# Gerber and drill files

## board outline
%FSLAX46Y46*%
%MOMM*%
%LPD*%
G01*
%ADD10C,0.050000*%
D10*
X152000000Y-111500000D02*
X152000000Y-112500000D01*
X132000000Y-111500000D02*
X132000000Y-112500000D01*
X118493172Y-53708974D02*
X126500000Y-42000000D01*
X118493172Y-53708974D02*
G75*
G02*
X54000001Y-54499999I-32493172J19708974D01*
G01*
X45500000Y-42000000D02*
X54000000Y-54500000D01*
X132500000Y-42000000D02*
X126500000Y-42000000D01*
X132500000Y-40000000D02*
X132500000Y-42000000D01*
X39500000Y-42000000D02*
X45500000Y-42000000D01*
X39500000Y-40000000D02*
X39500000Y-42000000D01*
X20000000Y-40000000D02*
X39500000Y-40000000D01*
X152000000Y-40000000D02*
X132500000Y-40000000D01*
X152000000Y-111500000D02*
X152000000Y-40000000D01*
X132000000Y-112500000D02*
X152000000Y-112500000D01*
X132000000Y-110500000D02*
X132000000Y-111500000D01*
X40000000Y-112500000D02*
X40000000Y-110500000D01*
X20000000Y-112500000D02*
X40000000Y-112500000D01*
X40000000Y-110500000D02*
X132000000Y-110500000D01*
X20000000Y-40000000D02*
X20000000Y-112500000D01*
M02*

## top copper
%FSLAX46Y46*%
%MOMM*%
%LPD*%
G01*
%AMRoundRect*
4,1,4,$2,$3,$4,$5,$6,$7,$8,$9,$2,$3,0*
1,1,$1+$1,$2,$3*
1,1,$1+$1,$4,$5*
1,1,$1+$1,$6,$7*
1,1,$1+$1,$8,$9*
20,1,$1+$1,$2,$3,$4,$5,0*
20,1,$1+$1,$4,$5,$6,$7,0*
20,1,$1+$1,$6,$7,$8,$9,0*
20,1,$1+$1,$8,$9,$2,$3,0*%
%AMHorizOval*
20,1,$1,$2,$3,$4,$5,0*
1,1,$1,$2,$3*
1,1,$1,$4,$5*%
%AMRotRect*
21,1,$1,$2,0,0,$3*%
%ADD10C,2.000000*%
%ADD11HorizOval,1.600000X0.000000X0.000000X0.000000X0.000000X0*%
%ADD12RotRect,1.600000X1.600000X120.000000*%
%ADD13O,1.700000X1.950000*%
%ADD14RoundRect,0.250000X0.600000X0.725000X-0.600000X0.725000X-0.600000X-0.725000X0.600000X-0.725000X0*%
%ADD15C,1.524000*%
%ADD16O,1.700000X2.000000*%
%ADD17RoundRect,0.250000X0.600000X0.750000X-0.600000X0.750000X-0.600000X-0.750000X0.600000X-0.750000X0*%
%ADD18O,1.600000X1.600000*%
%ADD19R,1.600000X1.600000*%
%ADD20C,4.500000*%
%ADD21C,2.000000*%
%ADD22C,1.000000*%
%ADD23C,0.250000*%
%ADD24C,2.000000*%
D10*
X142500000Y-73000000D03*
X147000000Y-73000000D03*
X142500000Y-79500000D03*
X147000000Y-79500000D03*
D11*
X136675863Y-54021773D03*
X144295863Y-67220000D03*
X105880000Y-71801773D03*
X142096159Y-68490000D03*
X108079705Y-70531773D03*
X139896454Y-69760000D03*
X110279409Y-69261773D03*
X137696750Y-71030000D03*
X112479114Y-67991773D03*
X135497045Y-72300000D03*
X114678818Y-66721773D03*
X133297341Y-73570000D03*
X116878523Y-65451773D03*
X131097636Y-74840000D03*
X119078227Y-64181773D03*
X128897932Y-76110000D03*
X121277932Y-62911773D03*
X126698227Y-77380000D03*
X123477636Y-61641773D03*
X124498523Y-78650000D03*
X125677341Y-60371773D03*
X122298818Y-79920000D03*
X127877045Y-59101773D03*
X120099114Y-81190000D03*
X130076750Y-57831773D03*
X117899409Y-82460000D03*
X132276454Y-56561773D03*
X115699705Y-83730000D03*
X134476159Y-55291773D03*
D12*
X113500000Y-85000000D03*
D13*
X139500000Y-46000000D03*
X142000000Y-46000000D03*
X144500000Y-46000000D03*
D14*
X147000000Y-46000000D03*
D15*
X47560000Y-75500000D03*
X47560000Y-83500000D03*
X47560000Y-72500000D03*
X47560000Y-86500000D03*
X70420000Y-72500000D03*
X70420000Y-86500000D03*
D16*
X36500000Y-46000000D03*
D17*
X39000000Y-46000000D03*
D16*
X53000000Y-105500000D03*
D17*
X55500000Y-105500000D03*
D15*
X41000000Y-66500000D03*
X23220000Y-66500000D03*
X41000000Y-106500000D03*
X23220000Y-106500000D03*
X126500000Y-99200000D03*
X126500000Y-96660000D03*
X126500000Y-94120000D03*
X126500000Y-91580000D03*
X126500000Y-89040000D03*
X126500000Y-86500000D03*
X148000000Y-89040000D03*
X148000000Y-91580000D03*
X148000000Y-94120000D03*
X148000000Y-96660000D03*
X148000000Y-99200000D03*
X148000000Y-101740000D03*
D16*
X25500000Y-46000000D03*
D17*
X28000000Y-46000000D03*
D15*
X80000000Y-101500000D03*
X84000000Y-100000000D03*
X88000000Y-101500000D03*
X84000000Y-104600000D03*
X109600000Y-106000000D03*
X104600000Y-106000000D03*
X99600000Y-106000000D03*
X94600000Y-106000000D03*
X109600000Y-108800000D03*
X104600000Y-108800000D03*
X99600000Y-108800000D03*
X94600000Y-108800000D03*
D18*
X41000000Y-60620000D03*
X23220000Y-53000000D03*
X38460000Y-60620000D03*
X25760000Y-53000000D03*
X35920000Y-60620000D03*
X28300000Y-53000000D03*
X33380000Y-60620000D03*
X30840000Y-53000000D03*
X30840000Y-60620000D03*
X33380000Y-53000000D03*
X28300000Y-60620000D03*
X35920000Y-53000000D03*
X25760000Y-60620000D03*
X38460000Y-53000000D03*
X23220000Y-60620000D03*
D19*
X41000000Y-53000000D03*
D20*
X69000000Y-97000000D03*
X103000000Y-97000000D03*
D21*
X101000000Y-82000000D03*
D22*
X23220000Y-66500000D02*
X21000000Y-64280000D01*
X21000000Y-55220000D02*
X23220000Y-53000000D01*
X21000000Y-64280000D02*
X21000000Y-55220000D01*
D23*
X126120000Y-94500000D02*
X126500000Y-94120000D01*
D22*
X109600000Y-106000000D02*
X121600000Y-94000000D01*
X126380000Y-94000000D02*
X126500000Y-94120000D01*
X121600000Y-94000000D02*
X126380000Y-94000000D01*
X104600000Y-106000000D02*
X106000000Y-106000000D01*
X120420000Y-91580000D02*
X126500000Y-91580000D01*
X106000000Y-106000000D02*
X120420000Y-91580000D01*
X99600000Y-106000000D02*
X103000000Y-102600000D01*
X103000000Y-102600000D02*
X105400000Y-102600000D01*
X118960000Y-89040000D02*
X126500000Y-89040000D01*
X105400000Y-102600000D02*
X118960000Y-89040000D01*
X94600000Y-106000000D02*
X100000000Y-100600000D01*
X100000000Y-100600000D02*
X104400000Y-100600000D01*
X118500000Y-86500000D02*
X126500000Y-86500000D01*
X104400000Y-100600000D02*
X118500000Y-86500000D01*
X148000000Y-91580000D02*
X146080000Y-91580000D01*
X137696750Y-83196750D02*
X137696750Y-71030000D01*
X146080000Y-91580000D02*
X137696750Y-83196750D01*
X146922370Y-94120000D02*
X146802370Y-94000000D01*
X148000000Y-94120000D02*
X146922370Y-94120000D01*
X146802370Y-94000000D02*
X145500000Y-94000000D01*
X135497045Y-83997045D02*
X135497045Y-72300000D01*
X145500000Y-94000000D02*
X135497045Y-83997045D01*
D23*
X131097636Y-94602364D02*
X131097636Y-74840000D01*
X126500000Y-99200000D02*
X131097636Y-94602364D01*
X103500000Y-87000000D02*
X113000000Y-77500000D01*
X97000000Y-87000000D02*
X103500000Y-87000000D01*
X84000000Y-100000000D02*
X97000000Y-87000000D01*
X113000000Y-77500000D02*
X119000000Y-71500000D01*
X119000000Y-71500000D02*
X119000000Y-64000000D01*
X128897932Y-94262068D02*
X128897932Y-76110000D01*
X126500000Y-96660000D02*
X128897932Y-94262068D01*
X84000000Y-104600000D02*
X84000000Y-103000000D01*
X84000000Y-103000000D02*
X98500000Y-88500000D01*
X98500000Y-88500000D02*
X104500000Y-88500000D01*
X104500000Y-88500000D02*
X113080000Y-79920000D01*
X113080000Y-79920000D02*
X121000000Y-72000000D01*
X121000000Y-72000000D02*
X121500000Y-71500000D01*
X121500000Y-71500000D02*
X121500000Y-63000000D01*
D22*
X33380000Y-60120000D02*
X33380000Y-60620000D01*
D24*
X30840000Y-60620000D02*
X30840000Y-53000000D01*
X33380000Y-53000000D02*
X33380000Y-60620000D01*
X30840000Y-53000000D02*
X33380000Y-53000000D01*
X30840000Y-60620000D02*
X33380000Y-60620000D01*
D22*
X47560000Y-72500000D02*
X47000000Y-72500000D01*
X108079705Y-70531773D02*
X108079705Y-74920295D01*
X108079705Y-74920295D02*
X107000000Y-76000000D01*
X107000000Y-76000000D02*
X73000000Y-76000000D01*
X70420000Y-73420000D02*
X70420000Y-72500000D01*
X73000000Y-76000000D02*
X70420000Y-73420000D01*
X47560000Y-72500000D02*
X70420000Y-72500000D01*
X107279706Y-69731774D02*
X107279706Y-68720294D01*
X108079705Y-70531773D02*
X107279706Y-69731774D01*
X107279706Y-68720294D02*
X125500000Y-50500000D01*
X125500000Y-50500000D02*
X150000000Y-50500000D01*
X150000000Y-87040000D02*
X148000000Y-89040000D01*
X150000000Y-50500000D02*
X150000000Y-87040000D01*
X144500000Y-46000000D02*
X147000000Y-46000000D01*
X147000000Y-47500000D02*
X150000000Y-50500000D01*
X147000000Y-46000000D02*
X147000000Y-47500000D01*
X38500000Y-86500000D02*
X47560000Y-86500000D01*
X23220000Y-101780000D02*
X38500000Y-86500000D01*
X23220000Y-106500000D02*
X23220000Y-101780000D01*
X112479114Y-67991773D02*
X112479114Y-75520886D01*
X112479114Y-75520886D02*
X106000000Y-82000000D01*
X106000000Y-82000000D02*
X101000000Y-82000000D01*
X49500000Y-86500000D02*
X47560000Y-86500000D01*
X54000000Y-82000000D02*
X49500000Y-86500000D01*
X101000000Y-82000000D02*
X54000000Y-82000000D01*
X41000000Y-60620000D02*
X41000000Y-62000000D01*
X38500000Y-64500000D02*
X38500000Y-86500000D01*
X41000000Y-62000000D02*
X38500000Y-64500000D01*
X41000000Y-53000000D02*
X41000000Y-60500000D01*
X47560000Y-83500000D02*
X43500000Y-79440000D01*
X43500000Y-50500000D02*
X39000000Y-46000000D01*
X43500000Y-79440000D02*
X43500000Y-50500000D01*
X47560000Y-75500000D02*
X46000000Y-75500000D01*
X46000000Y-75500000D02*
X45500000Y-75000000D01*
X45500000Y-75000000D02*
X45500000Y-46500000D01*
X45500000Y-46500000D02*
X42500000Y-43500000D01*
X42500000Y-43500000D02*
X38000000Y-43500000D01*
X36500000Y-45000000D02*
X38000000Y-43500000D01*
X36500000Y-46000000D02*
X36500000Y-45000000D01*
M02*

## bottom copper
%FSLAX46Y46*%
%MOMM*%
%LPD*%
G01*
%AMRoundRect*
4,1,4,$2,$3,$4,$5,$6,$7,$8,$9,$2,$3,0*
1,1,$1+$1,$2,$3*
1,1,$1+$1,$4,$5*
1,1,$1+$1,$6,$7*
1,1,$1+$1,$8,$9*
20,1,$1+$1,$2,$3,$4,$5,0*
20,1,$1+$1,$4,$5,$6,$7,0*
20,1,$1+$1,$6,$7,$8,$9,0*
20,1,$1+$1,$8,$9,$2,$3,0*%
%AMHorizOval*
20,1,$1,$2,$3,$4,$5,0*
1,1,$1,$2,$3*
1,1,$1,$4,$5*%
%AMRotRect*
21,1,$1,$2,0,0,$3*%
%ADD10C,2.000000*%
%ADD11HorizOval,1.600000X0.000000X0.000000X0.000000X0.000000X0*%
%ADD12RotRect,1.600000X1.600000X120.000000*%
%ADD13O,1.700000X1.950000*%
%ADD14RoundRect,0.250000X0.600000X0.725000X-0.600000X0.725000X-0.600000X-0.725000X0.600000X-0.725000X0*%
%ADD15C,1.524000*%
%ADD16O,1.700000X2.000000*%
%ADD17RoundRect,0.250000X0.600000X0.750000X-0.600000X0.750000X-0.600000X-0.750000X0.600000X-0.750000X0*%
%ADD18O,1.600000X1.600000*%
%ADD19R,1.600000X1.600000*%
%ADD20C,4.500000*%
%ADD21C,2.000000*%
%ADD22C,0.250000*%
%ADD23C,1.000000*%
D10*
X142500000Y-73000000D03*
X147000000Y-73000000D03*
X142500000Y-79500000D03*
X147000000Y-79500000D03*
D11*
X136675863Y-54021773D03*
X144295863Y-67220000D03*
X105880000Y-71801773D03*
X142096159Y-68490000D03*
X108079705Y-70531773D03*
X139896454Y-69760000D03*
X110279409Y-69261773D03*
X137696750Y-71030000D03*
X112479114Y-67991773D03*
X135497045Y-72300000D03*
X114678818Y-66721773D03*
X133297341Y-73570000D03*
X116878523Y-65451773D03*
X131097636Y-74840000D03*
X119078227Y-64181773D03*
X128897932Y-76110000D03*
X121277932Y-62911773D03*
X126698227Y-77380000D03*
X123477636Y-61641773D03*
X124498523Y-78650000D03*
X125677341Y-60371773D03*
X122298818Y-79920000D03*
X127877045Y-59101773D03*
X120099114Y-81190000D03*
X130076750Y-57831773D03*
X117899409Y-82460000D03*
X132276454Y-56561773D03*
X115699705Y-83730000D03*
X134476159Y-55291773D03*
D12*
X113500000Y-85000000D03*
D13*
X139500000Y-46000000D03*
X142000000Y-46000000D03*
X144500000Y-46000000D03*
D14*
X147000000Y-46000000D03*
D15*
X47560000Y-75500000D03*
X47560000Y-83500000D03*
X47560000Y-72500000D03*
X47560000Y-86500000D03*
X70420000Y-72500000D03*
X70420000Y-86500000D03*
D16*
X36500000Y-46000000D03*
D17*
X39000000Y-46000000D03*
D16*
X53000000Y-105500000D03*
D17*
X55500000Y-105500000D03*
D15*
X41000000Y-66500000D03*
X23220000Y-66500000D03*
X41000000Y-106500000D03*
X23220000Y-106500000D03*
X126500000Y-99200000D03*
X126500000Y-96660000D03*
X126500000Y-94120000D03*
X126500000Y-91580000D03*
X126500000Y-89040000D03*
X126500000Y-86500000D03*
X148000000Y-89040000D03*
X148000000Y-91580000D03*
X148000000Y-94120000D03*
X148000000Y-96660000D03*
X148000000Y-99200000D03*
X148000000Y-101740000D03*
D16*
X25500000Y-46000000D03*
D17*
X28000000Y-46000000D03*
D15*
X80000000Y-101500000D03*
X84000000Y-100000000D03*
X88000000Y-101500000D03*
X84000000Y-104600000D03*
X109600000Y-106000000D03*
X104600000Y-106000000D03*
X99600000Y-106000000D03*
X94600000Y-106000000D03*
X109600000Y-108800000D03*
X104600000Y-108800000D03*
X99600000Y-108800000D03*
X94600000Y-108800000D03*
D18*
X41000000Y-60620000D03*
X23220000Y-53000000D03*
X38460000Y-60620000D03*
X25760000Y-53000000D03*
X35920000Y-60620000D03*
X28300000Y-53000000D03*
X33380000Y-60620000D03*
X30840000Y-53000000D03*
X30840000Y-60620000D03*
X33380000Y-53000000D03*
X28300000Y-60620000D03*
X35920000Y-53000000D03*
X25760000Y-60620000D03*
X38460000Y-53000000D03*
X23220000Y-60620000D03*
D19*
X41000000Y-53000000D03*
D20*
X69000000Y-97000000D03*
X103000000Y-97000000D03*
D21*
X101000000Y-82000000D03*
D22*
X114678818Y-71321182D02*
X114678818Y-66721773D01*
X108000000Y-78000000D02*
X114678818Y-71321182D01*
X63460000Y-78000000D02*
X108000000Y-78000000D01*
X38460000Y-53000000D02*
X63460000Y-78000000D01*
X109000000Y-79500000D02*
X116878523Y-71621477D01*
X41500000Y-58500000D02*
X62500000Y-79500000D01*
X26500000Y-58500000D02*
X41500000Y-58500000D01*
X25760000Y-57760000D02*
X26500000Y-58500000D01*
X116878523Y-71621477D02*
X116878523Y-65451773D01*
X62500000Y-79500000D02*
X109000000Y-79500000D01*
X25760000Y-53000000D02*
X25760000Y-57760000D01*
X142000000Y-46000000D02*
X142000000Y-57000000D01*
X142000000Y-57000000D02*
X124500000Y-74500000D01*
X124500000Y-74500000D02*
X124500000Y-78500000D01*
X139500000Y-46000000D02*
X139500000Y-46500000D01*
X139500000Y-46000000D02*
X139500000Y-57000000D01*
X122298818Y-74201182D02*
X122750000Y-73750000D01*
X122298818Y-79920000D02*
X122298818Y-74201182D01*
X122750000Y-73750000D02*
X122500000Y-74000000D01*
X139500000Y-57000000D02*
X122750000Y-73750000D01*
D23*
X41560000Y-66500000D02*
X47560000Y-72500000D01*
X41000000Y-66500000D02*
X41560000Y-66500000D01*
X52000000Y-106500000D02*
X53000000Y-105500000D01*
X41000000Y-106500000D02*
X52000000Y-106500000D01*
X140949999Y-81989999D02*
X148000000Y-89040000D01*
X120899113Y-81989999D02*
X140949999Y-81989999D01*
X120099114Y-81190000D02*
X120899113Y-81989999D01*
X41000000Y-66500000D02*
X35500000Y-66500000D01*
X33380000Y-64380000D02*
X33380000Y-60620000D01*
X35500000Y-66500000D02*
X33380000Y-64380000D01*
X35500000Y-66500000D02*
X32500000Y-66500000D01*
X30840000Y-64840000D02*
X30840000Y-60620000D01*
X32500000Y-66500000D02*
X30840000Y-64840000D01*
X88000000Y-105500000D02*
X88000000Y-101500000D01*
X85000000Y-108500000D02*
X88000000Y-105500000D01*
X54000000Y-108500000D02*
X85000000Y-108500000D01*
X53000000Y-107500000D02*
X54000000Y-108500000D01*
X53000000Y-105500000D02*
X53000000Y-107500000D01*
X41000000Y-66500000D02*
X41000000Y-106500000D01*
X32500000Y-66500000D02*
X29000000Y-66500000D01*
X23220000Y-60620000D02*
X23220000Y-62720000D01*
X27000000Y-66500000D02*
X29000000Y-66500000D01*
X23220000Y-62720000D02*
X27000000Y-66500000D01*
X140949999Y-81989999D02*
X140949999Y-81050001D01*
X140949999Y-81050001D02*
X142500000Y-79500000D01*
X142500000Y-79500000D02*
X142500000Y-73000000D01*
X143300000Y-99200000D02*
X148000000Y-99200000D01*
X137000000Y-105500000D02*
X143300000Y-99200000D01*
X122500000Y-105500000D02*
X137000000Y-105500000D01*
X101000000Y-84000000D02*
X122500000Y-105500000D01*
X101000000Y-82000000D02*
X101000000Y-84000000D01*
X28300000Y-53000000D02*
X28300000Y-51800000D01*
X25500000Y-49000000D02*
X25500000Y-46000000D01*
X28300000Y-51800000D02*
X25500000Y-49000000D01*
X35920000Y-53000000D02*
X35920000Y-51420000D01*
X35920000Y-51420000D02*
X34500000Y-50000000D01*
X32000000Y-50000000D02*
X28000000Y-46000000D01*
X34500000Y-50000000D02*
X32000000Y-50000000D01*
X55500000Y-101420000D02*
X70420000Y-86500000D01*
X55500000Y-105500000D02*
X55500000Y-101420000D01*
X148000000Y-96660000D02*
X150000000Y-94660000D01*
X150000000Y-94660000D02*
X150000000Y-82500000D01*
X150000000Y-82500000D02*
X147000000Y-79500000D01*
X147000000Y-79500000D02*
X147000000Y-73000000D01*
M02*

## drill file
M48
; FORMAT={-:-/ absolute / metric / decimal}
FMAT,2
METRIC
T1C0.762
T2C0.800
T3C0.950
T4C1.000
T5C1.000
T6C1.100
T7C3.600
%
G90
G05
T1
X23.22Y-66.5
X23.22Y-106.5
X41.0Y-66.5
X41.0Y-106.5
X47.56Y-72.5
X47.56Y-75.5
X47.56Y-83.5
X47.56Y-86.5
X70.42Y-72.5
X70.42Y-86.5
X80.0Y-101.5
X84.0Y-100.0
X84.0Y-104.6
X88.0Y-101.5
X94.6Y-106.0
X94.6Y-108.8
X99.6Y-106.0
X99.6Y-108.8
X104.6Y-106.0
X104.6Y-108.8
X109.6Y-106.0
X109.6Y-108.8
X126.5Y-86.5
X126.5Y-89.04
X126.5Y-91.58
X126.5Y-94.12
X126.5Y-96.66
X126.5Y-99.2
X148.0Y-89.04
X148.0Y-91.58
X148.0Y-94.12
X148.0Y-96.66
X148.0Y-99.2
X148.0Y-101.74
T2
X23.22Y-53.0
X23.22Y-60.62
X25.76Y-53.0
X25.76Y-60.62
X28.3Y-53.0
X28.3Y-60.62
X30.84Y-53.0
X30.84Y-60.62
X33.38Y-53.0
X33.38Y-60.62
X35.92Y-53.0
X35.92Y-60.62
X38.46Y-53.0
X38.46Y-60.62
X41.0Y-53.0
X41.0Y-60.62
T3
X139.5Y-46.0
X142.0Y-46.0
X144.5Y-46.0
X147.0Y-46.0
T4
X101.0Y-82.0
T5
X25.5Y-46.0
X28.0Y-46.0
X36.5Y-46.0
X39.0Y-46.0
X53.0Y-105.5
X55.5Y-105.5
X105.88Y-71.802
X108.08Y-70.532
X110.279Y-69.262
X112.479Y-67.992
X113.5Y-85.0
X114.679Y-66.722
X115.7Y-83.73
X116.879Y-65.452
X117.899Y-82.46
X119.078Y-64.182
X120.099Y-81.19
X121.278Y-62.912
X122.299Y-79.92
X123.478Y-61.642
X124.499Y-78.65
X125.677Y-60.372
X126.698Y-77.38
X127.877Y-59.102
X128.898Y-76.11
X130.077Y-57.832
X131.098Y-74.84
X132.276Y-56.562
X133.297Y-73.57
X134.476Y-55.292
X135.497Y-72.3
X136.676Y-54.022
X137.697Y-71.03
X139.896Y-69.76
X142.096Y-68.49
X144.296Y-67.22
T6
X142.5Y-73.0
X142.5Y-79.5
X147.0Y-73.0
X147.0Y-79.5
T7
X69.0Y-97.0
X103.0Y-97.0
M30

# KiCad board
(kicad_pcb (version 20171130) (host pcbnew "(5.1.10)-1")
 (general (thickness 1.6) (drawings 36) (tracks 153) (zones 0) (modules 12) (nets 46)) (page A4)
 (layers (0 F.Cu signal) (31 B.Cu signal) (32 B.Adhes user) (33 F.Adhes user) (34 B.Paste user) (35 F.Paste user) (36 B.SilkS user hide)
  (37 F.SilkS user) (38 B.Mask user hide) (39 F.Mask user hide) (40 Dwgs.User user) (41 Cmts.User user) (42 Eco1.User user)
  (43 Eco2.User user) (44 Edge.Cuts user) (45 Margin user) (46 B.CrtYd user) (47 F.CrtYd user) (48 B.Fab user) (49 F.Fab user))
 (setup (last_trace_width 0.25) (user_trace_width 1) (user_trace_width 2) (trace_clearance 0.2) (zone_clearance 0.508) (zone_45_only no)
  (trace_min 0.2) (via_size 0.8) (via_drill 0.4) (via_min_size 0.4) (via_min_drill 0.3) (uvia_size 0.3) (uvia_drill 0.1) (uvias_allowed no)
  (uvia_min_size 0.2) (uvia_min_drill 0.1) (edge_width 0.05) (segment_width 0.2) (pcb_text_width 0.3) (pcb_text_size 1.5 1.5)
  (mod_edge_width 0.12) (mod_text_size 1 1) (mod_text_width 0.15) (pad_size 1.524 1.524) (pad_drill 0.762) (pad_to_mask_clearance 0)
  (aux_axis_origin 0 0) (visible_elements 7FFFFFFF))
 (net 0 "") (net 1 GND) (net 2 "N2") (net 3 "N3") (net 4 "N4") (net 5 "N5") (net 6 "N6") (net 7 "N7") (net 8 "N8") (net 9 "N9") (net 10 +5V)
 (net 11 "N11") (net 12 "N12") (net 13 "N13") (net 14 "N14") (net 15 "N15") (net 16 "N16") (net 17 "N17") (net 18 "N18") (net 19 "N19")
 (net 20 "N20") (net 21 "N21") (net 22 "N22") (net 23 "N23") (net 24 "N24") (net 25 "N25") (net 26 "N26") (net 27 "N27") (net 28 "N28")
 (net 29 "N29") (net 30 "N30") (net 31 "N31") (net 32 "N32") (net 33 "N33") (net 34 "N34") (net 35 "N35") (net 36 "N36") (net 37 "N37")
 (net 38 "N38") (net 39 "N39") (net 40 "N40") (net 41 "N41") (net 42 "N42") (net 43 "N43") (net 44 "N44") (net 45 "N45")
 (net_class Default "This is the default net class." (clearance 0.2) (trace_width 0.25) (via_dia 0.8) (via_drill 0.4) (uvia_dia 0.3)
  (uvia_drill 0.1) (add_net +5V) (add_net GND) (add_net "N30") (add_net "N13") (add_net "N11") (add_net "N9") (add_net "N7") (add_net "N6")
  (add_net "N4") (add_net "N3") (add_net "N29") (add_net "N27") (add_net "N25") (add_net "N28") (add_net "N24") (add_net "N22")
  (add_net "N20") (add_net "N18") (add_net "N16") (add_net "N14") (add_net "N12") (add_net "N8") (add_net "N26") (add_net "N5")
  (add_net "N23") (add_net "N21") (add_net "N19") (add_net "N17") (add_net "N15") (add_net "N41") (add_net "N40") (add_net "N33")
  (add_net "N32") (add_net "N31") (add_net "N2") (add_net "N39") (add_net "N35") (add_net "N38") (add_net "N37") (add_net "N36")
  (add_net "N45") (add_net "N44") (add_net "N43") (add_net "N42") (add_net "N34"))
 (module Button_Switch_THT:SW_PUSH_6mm (layer F.Cu) (at 142.5 79.5 90)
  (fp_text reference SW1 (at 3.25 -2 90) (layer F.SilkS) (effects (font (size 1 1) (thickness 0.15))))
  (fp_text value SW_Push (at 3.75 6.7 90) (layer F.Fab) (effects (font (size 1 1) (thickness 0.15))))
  (pad 1 thru_hole circle (at 6.5 0 180) (size 2 2) (drill 1.1) (layers *.Cu *.Mask) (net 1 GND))
  (pad 2 thru_hole circle (at 6.5 4.5 180) (size 2 2) (drill 1.1) (layers *.Cu *.Mask) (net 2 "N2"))
  (pad 1 thru_hole circle (at 0 0 180) (size 2 2) (drill 1.1) (layers *.Cu *.Mask) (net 1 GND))
  (pad 2 thru_hole circle (at 0 4.5 180) (size 2 2) (drill 1.1) (layers *.Cu *.Mask) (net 2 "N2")))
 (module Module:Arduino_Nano (layer F.Cu) (at 113.5 85 120)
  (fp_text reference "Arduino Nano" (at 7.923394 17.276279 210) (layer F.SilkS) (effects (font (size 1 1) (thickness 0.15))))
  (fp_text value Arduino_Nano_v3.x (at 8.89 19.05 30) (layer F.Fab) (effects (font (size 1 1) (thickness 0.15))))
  (pad 16 thru_hole oval (at 15.24 35.56 120) (size 1.6 1.6) (drill 1) (layers *.Cu *.Mask) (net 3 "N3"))
  (pad 15 thru_hole oval (at 0 35.56 120) (size 1.6 1.6) (drill 1) (layers *.Cu *.Mask) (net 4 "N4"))
  (pad 30 thru_hole oval (at 15.24 0 120) (size 1.6 1.6) (drill 1) (layers *.Cu *.Mask) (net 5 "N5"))
  (pad 14 thru_hole oval (at 0 33.02 120) (size 1.6 1.6) (drill 1) (layers *.Cu *.Mask) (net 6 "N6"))
  (pad 29 thru_hole oval (at 15.24 2.54 120) (size 1.6 1.6) (drill 1) (layers *.Cu *.Mask) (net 1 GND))
  (pad 13 thru_hole oval (at 0 30.48 120) (size 1.6 1.6) (drill 1) (layers *.Cu *.Mask) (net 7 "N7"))
  (pad 28 thru_hole oval (at 15.24 5.08 120) (size 1.6 1.6) (drill 1) (layers *.Cu *.Mask) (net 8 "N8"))
  (pad 12 thru_hole oval (at 0 27.94 120) (size 1.6 1.6) (drill 1) (layers *.Cu *.Mask) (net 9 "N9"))
  (pad 27 thru_hole oval (at 15.24 7.62 120) (size 1.6 1.6) (drill 1) (layers *.Cu *.Mask) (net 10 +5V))
  (pad 11 thru_hole oval (at 0 25.4 120) (size 1.6 1.6) (drill 1) (layers *.Cu *.Mask) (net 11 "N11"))
  (pad 26 thru_hole oval (at 15.24 10.16 120) (size 1.6 1.6) (drill 1) (layers *.Cu *.Mask) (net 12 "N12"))
  (pad 10 thru_hole oval (at 0 22.86 120) (size 1.6 1.6) (drill 1) (layers *.Cu *.Mask) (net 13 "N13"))
  (pad 25 thru_hole oval (at 15.24 12.7 120) (size 1.6 1.6) (drill 1) (layers *.Cu *.Mask) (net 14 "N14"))
  (pad 9 thru_hole oval (at 0 20.32 120) (size 1.6 1.6) (drill 1) (layers *.Cu *.Mask) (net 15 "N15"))
  (pad 24 thru_hole oval (at 15.24 15.24 120) (size 1.6 1.6) (drill 1) (layers *.Cu *.Mask) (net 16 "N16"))
  (pad 8 thru_hole oval (at 0 17.78 120) (size 1.6 1.6) (drill 1) (layers *.Cu *.Mask) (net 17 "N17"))
  (pad 23 thru_hole oval (at 15.24 17.78 120) (size 1.6 1.6) (drill 1) (layers *.Cu *.Mask) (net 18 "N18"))
  (pad 7 thru_hole oval (at 0 15.24 120) (size 1.6 1.6) (drill 1) (layers *.Cu *.Mask) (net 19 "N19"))
  (pad 22 thru_hole oval (at 15.24 20.32 120) (size 1.6 1.6) (drill 1) (layers *.Cu *.Mask) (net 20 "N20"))
  (pad 6 thru_hole oval (at 0 12.7 120) (size 1.6 1.6) (drill 1) (layers *.Cu *.Mask) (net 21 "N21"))
  (pad 21 thru_hole oval (at 15.24 22.86 120) (size 1.6 1.6) (drill 1) (layers *.Cu *.Mask) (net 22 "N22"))
  (pad 5 thru_hole oval (at 0 10.16 120) (size 1.6 1.6) (drill 1) (layers *.Cu *.Mask) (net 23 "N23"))
  (pad 20 thru_hole oval (at 15.24 25.4 120) (size 1.6 1.6) (drill 1) (layers *.Cu *.Mask) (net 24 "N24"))
  (pad 4 thru_hole oval (at 0 7.62 120) (size 1.6 1.6) (drill 1) (layers *.Cu *.Mask) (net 1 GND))
  (pad 19 thru_hole oval (at 15.24 27.94 120) (size 1.6 1.6) (drill 1) (layers *.Cu *.Mask) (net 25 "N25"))
  (pad 3 thru_hole oval (at 0 5.08 120) (size 1.6 1.6) (drill 1) (layers *.Cu *.Mask) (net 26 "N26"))
  (pad 18 thru_hole oval (at 15.24 30.48 120) (size 1.6 1.6) (drill 1) (layers *.Cu *.Mask) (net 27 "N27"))
  (pad 2 thru_hole oval (at 0 2.54 120) (size 1.6 1.6) (drill 1) (layers *.Cu *.Mask) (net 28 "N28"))
  (pad 17 thru_hole oval (at 15.24 33.02 120) (size 1.6 1.6) (drill 1) (layers *.Cu *.Mask) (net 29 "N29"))
  (pad 1 thru_hole rect (at 0 0 120) (size 1.6 1.6) (drill 1) (layers *.Cu *.Mask) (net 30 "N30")))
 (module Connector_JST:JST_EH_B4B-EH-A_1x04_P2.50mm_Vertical (layer F.Cu) (at 147 46 180)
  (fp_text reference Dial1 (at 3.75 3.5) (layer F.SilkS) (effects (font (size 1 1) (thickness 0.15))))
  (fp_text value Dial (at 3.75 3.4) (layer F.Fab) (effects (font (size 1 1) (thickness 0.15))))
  (pad 4 thru_hole oval (at 7.5 0 180) (size 1.7 1.95) (drill 0.95) (layers *.Cu *.Mask) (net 23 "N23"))
  (pad 3 thru_hole oval (at 5 0 180) (size 1.7 1.95) (drill 0.95) (layers *.Cu *.Mask) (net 21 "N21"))
  (pad 2 thru_hole oval (at 2.5 0 180) (size 1.7 1.95) (drill 0.95) (layers *.Cu *.Mask) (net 1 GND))
  (pad 1 thru_hole roundrect (at 0 0 180) (size 1.7 1.95) (drill 0.95) (layers *.Cu *.Mask) (roundrect_rratio 0.1470588235294118)
   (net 1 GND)))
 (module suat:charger (layer F.Cu) (at 75.5 72.5 180)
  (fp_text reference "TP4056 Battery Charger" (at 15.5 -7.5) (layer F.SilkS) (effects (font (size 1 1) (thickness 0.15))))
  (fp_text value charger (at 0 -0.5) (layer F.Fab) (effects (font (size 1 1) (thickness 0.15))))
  (pad 6 thru_hole circle (at 27.94 -3 180) (size 1.524 1.524) (drill 0.762) (layers *.Cu *.Mask) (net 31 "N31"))
  (pad 5 thru_hole circle (at 27.94 -11 180) (size 1.524 1.524) (drill 0.762) (layers *.Cu *.Mask) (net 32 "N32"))
  (pad 4 thru_hole circle (at 27.94 0 180) (size 1.524 1.524) (drill 0.762) (layers *.Cu *.Mask) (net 1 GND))
  (pad 3 thru_hole circle (at 27.94 -14 180) (size 1.524 1.524) (drill 0.762) (layers *.Cu *.Mask) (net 10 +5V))
  (pad 2 thru_hole circle (at 5.08 0 180) (size 1.524 1.524) (drill 0.762) (layers *.Cu *.Mask) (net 1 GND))
  (pad 1 thru_hole circle (at 5.08 -14 180) (size 1.524 1.524) (drill 0.762) (layers *.Cu *.Mask) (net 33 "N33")))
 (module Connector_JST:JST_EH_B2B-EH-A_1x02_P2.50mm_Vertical (layer F.Cu) (at 39 46 180)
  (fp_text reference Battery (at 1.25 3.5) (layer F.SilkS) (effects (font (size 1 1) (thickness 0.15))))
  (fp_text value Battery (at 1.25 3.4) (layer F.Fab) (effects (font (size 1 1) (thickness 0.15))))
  (pad 2 thru_hole oval (at 2.5 0 180) (size 1.7 2) (drill 1) (layers *.Cu *.Mask) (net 31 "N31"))
  (pad 1 thru_hole roundrect (at 0 0 180) (size 1.7 2) (drill 1) (layers *.Cu *.Mask) (roundrect_rratio 0.1470588235294118) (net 32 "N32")))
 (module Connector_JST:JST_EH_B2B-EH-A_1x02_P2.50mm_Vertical (layer F.Cu) (at 55.5 105.5 180)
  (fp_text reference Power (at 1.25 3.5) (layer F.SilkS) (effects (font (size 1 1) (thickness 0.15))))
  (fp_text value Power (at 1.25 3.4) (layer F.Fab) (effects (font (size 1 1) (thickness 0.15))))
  (pad 2 thru_hole oval (at 2.5 0 180) (size 1.7 2) (drill 1) (layers *.Cu *.Mask) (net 1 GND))
  (pad 1 thru_hole roundrect (at 0 0 180) (size 1.7 2) (drill 1) (layers *.Cu *.Mask) (roundrect_rratio 0.1470588235294118) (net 33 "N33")))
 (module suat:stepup (layer F.Cu) (at 41 106.5 90)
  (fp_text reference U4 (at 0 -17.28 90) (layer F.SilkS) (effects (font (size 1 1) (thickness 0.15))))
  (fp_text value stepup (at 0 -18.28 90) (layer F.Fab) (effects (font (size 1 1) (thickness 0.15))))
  (pad 4 thru_hole circle (at 40 0 90) (size 1.524 1.524) (drill 0.762) (layers *.Cu *.Mask) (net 1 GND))
  (pad 3 thru_hole circle (at 40 -17.78 90) (size 1.524 1.524) (drill 0.762) (layers *.Cu *.Mask) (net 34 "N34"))
  (pad 2 thru_hole circle (at 0 0 90) (size 1.524 1.524) (drill 0.762) (layers *.Cu *.Mask) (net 1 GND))
  (pad 1 thru_hole circle (at 0 -17.78 90) (size 1.524 1.524) (drill 0.762) (layers *.Cu *.Mask) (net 10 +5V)))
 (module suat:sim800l (layer F.Cu) (at 148 86.5 180)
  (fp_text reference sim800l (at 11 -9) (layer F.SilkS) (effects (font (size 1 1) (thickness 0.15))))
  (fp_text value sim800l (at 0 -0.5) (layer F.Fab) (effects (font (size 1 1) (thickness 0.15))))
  (pad 12 thru_hole circle (at 21.5 -12.7 180) (size 1.524 1.524) (drill 0.762) (layers *.Cu *.Mask) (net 15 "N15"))
  (pad 11 thru_hole circle (at 21.5 -10.16 180) (size 1.524 1.524) (drill 0.762) (layers *.Cu *.Mask) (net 17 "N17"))
  (pad 10 thru_hole circle (at 21.5 -7.62 180) (size 1.524 1.524) (drill 0.762) (layers *.Cu *.Mask) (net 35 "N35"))
  (pad 9 thru_hole circle (at 21.5 -5.08 180) (size 1.524 1.524) (drill 0.762) (layers *.Cu *.Mask) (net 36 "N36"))
  (pad 8 thru_hole circle (at 21.5 -2.54 180) (size 1.524 1.524) (drill 0.762) (layers *.Cu *.Mask) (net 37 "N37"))
  (pad 7 thru_hole circle (at 21.5 0 180) (size 1.524 1.524) (drill 0.762) (layers *.Cu *.Mask) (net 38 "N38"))
  (pad 6 thru_hole circle (at 0 -2.54 180) (size 1.524 1.524) (drill 0.762) (layers *.Cu *.Mask) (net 1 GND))
  (pad 5 thru_hole circle (at 0 -5.08 180) (size 1.524 1.524) (drill 0.762) (layers *.Cu *.Mask) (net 9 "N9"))
  (pad 4 thru_hole circle (at 0 -7.62 180) (size 1.524 1.524) (drill 0.762) (layers *.Cu *.Mask) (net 11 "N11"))
  (pad 3 thru_hole circle (at 0 -10.16 180) (size 1.524 1.524) (drill 0.762) (layers *.Cu *.Mask) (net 2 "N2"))
  (pad 2 thru_hole circle (at 0 -12.7 180) (size 1.524 1.524) (drill 0.762) (layers *.Cu *.Mask) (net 10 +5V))
  (pad 1 thru_hole circle (at 0 -15.24 180) (size 1.524 1.524) (drill 0.762) (layers *.Cu *.Mask) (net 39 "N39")))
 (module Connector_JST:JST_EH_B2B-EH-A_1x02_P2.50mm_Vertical (layer F.Cu) (at 28 46 180)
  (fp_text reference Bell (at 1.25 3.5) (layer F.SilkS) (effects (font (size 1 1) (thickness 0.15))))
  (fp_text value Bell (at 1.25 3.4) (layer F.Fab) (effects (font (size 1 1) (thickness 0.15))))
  (pad 2 thru_hole oval (at 2.5 0 180) (size 1.7 2) (drill 1) (layers *.Cu *.Mask) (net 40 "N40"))
  (pad 1 thru_hole roundrect (at 0 0 180) (size 1.7 2) (drill 1) (layers *.Cu *.Mask) (roundrect_rratio 0.1470588235294118) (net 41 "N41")))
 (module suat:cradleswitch (layer F.Cu) (at 84 104.7)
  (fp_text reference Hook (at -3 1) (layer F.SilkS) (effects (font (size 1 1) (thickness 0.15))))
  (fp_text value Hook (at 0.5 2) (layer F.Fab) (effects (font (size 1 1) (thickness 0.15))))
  (pad 4 thru_hole circle (at -4 -3.2) (size 1.524 1.524) (drill 0.762) (layers *.Cu *.Mask))
  (pad 3 thru_hole circle (at 0 -4.7) (size 1.524 1.524) (drill 0.762) (layers *.Cu *.Mask) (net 16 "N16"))
  (pad 2 thru_hole circle (at 4 -3.2) (size 1.524 1.524) (drill 0.762) (layers *.Cu *.Mask) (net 1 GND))
  (pad 1 thru_hole circle (at 0 -0.1) (size 1.524 1.524) (drill 0.762) (layers *.Cu *.Mask) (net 18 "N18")))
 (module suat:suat (layer F.Cu) (at 109.6 106)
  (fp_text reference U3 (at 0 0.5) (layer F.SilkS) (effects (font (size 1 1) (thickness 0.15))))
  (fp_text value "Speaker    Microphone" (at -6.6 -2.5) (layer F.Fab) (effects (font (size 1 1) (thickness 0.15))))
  (pad 1 thru_hole circle (at 0 0) (size 1.524 1.524) (drill 0.762) (layers *.Cu *.Mask) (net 35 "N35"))
  (pad 2 thru_hole circle (at -5 0) (size 1.524 1.524) (drill 0.762) (layers *.Cu *.Mask) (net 36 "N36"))
  (pad 3 thru_hole circle (at -10 0) (size 1.524 1.524) (drill 0.762) (layers *.Cu *.Mask) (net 37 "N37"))
  (pad 4 thru_hole circle (at -15 0) (size 1.524 1.524) (drill 0.762) (layers *.Cu *.Mask) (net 38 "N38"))
  (pad 5 thru_hole circle (at 0 2.8) (size 1.524 1.524) (drill 0.762) (layers *.Cu *.Mask))
  (pad 6 thru_hole circle (at -5 2.8) (size 1.524 1.524) (drill 0.762) (layers *.Cu *.Mask))
  (pad 7 thru_hole circle (at -10 2.8) (size 1.524 1.524) (drill 0.762) (layers *.Cu *.Mask))
  (pad 8 thru_hole circle (at -15 2.8) (size 1.524 1.524) (drill 0.762) (layers *.Cu *.Mask)))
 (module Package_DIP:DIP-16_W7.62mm (layer F.Cu) (at 41 53 270)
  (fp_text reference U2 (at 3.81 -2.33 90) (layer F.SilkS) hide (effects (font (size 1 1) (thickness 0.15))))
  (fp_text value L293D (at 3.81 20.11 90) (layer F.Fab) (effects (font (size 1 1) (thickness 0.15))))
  (pad 16 thru_hole oval (at 7.62 0 270) (size 1.6 1.6) (drill 0.8) (layers *.Cu *.Mask) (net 10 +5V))
  (pad 8 thru_hole oval (at 0 17.78 270) (size 1.6 1.6) (drill 0.8) (layers *.Cu *.Mask) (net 34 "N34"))
  (pad 15 thru_hole oval (at 7.62 2.54 270) (size 1.6 1.6) (drill 0.8) (layers *.Cu *.Mask) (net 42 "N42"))
  (pad 7 thru_hole oval (at 0 15.24 270) (size 1.6 1.6) (drill 0.8) (layers *.Cu *.Mask) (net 14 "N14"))
  (pad 14 thru_hole oval (at 7.62 5.08 270) (size 1.6 1.6) (drill 0.8) (layers *.Cu *.Mask) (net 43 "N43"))
  (pad 6 thru_hole oval (at 0 12.7 270) (size 1.6 1.6) (drill 0.8) (layers *.Cu *.Mask) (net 40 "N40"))
  (pad 13 thru_hole oval (at 7.62 7.62 270) (size 1.6 1.6) (drill 0.8) (layers *.Cu *.Mask) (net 1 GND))
  (pad 5 thru_hole oval (at 0 10.16 270) (size 1.6 1.6) (drill 0.8) (layers *.Cu *.Mask) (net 1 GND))
  (pad 12 thru_hole oval (at 7.62 10.16 270) (size 1.6 1.6) (drill 0.8) (layers *.Cu *.Mask) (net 1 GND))
  (pad 4 thru_hole oval (at 0 7.62 270) (size 1.6 1.6) (drill 0.8) (layers *.Cu *.Mask) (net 1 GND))
  (pad 11 thru_hole oval (at 7.62 12.7 270) (size 1.6 1.6) (drill 0.8) (layers *.Cu *.Mask) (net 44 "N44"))
  (pad 3 thru_hole oval (at 0 5.08 270) (size 1.6 1.6) (drill 0.8) (layers *.Cu *.Mask) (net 41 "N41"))
  (pad 10 thru_hole oval (at 7.62 15.24 270) (size 1.6 1.6) (drill 0.8) (layers *.Cu *.Mask) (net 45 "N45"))
  (pad 2 thru_hole oval (at 0 2.54 270) (size 1.6 1.6) (drill 0.8) (layers *.Cu *.Mask) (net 12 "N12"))
  (pad 9 thru_hole oval (at 7.62 17.78 270) (size 1.6 1.6) (drill 0.8) (layers *.Cu *.Mask) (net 1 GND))
  (pad 1 thru_hole rect (at 0 0 270) (size 1.6 1.6) (drill 0.8) (layers *.Cu *.Mask) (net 10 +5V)))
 (gr_line (start 152 111.5) (end 152 112.5) (layer Edge.Cuts) (width 0.05))
 (gr_line (start 132 111.5) (end 132 112.5) (layer Edge.Cuts) (width 0.05))
 (gr_line (start 118.493172 53.708974) (end 126.5 42) (layer Edge.Cuts) (width 0.05))
 (gr_arc (start 86 34) (end 54.000001 54.499999) (angle -116.116145) (layer Edge.Cuts) (width 0.05))
 (gr_line (start 45.5 42) (end 54 54.5) (layer Edge.Cuts) (width 0.05))
 (gr_line (start 132.5 42) (end 126.5 42) (layer Edge.Cuts) (width 0.05))
 (gr_line (start 132.5 40) (end 132.5 42) (layer Edge.Cuts) (width 0.05))
 (gr_line (start 39.5 42) (end 45.5 42) (layer Edge.Cuts) (width 0.05))
 (gr_line (start 39.5 40) (end 39.5 42) (layer Edge.Cuts) (width 0.05))
 (gr_line (start 20 40) (end 39.5 40) (layer Edge.Cuts) (width 0.05))
 (gr_line (start 152 40) (end 132.5 40) (layer Edge.Cuts) (width 0.05))
 (gr_line (start 152 111.5) (end 152 40) (layer Edge.Cuts) (width 0.05))
 (gr_line (start 132 112.5) (end 152 112.5) (layer Edge.Cuts) (width 0.05))
 (gr_line (start 132 110.5) (end 132 111.5) (layer Edge.Cuts) (width 0.05))
 (gr_line (start 40 112.5) (end 40 110.5) (layer Edge.Cuts) (width 0.05))
 (gr_line (start 20 112.5) (end 40 112.5) (layer Edge.Cuts) (width 0.05))
 (gr_line (start 40 110.5) (end 132 110.5) (layer Edge.Cuts) (width 0.05))
 (gr_line (start 20 40) (end 20 112.5) (layer Edge.Cuts) (width 0.05))
 (via (at 69 97) (size 4.5) (drill 3.6) (layers F.Cu B.Cu) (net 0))
 (via (at 103 97) (size 4.5) (drill 3.6) (layers F.Cu B.Cu) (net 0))
 (segment (start 23.22 66.5) (end 21 64.28) (width 1) (layer F.Cu) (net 34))
 (segment (start 21 55.22) (end 23.22 53) (width 1) (layer F.Cu) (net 34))
 (segment (start 21 64.28) (end 21 55.22) (width 1) (layer F.Cu) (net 34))
 (segment (start 126.12 94.5) (end 126.5 94.12) (width 0.25) (layer F.Cu) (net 35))
 (segment (start 109.6 106) (end 121.6 94) (width 1) (layer F.Cu) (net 35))
 (segment (start 126.38 94) (end 126.5 94.12) (width 1) (layer F.Cu) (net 35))
 (segment (start 121.6 94) (end 126.38 94) (width 1) (layer F.Cu) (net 35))
 (segment (start 104.6 106) (end 106 106) (width 1) (layer F.Cu) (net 36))
 (segment (start 120.42 91.58) (end 126.5 91.58) (width 1) (layer F.Cu) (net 36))
 (segment (start 106 106) (end 120.42 91.58) (width 1) (layer F.Cu) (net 36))
 (segment (start 99.6 106) (end 103 102.6) (width 1) (layer F.Cu) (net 37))
 (segment (start 103 102.6) (end 105.4 102.6) (width 1) (layer F.Cu) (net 37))
 (segment (start 118.96 89.04) (end 126.5 89.04) (width 1) (layer F.Cu) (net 37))
 (segment (start 105.4 102.6) (end 118.96 89.04) (width 1) (layer F.Cu) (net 37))
 (segment (start 94.6 106) (end 100 100.6) (width 1) (layer F.Cu) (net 38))
 (segment (start 100 100.6) (end 104.4 100.6) (width 1) (layer F.Cu) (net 38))
 (segment (start 118.5 86.5) (end 126.5 86.5) (width 1) (layer F.Cu) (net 38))
 (segment (start 104.4 100.6) (end 118.5 86.5) (width 1) (layer F.Cu) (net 38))
 (segment (start 148 91.58) (end 146.08 91.58) (width 1) (layer F.Cu) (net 9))
 (segment (start 137.69675 83.19675) (end 137.69675 71.03) (width 1) (layer F.Cu) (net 9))
 (segment (start 146.08 91.58) (end 137.69675 83.19675) (width 1) (layer F.Cu) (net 9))
 (segment (start 146.92237 94.12) (end 146.80237 94) (width 1) (layer F.Cu) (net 11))
 (segment (start 148 94.12) (end 146.92237 94.12) (width 1) (layer F.Cu) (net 11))
 (segment (start 146.80237 94) (end 145.5 94) (width 1) (layer F.Cu) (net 11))
 (segment (start 135.497045 83.997045) (end 135.497045 72.3) (width 1) (layer F.Cu) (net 11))
 (segment (start 145.5 94) (end 135.497045 83.997045) (width 1) (layer F.Cu) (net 11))
 (segment (start 114.678818 71.321182) (end 114.678818 66.721773) (width 0.25) (layer B.Cu) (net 12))
 (segment (start 108 78) (end 114.678818 71.321182) (width 0.25) (layer B.Cu) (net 12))
 (segment (start 63.46 78) (end 108 78) (width 0.25) (layer B.Cu) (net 12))
 (segment (start 38.46 53) (end 63.46 78) (width 0.25) (layer B.Cu) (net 12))
 (segment (start 109 79.5) (end 116.878523 71.621477) (width 0.25) (layer B.Cu) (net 14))
 (segment (start 41.5 58.5) (end 62.5 79.5) (width 0.25) (layer B.Cu) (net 14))
 (segment (start 26.5 58.5) (end 41.5 58.5) (width 0.25) (layer B.Cu) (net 14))
 (segment (start 25.76 57.76) (end 26.5 58.5) (width 0.25) (layer B.Cu) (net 14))
 (segment (start 116.878523 71.621477) (end 116.878523 65.451773) (width 0.25) (layer B.Cu) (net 14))
 (segment (start 62.5 79.5) (end 109 79.5) (width 0.25) (layer B.Cu) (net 14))
 (segment (start 25.76 53) (end 25.76 57.76) (width 0.25) (layer B.Cu) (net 14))
 (segment (start 131.097636 94.602364) (end 131.097636 74.84) (width 0.25) (layer F.Cu) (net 15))
 (segment (start 126.5 99.2) (end 131.097636 94.602364) (width 0.25) (layer F.Cu) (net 15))
 (segment (start 103.5 87) (end 113 77.5) (width 0.25) (layer F.Cu) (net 16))
 (segment (start 97 87) (end 103.5 87) (width 0.25) (layer F.Cu) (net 16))
 (segment (start 84 100) (end 97 87) (width 0.25) (layer F.Cu) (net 16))
 (segment (start 113 77.5) (end 119 71.5) (width 0.25) (layer F.Cu) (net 16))
 (segment (start 119 71.5) (end 119 64) (width 0.25) (layer F.Cu) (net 16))
 (segment (start 128.897932 94.262068) (end 128.897932 76.11) (width 0.25) (layer F.Cu) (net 17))
 (segment (start 126.5 96.66) (end 128.897932 94.262068) (width 0.25) (layer F.Cu) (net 17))
 (segment (start 84 104.6) (end 84 103) (width 0.25) (layer F.Cu) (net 18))
 (segment (start 84 103) (end 98.5 88.5) (width 0.25) (layer F.Cu) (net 18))
 (segment (start 98.5 88.5) (end 104.5 88.5) (width 0.25) (layer F.Cu) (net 18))
 (segment (start 104.5 88.5) (end 113.08 79.92) (width 0.25) (layer F.Cu) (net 18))
 (segment (start 113.08 79.92) (end 121 72) (width 0.25) (layer F.Cu) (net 18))
 (segment (start 121 72) (end 121.5 71.5) (width 0.25) (layer F.Cu) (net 18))
 (segment (start 121.5 71.5) (end 121.5 63) (width 0.25) (layer F.Cu) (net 18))
 (segment (start 142 46) (end 142 57) (width 0.25) (layer B.Cu) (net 21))
 (segment (start 142 57) (end 124.5 74.5) (width 0.25) (layer B.Cu) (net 21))
 (segment (start 124.5 74.5) (end 124.5 78.5) (width 0.25) (layer B.Cu) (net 21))
 (segment (start 139.5 46) (end 139.5 46.5) (width 0.25) (layer B.Cu) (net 23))
 (segment (start 139.5 46) (end 139.5 57) (width 0.25) (layer B.Cu) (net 23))
 (segment (start 122.298818 74.201182) (end 122.75 73.75) (width 0.25) (layer B.Cu) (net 23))
 (segment (start 122.298818 79.92) (end 122.298818 74.201182) (width 0.25) (layer B.Cu) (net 23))
 (segment (start 122.75 73.75) (end 122.5 74) (width 0.25) (layer B.Cu) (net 23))
 (segment (start 139.5 57) (end 122.75 73.75) (width 0.25) (layer B.Cu) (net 23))
 (segment (start 33.38 60.12) (end 33.38 60.62) (width 1) (layer F.Cu) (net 1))
 (segment (start 30.84 60.62) (end 30.84 53) (width 2) (layer F.Cu) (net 1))
 (segment (start 33.38 53) (end 33.38 60.62) (width 2) (layer F.Cu) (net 1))
 (segment (start 30.84 53) (end 33.38 53) (width 2) (layer F.Cu) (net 1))
 (segment (start 30.84 60.62) (end 33.38 60.62) (width 2) (layer F.Cu) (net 1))
 (segment (start 47.56 72.5) (end 47 72.5) (width 1) (layer F.Cu) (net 1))
 (segment (start 41.56 66.5) (end 47.56 72.5) (width 1) (layer B.Cu) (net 1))
 (segment (start 41 66.5) (end 41.56 66.5) (width 1) (layer B.Cu) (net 1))
 (segment (start 52 106.5) (end 53 105.5) (width 1) (layer B.Cu) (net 1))
 (segment (start 41 106.5) (end 52 106.5) (width 1) (layer B.Cu) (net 1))
 (segment (start 108.079705 70.531773) (end 108.079705 74.920295) (width 1) (layer F.Cu) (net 1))
 (segment (start 108.079705 74.920295) (end 107 76) (width 1) (layer F.Cu) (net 1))
 (segment (start 107 76) (end 73 76) (width 1) (layer F.Cu) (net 1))
 (segment (start 70.42 73.42) (end 70.42 72.5) (width 1) (layer F.Cu) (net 1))
 (segment (start 73 76) (end 70.42 73.42) (width 1) (layer F.Cu) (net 1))
 (segment (start 47.56 72.5) (end 70.42 72.5) (width 1) (layer F.Cu) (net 1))
 (segment (start 107.279706 69.731774) (end 107.279706 68.720294) (width 1) (layer F.Cu) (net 1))
 (segment (start 108.079705 70.531773) (end 107.279706 69.731774) (width 1) (layer F.Cu) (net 1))
 (segment (start 107.279706 68.720294) (end 125.5 50.5) (width 1) (layer F.Cu) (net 1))
 (segment (start 125.5 50.5) (end 150 50.5) (width 1) (layer F.Cu) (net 1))
 (segment (start 150 87.04) (end 148 89.04) (width 1) (layer F.Cu) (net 1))
 (segment (start 150 50.5) (end 150 87.04) (width 1) (layer F.Cu) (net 1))
 (segment (start 140.949999 81.989999) (end 148 89.04) (width 1) (layer B.Cu) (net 1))
 (segment (start 120.899113 81.989999) (end 140.949999 81.989999) (width 1) (layer B.Cu) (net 1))
 (segment (start 120.099114 81.19) (end 120.899113 81.989999) (width 1) (layer B.Cu) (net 1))
 (segment (start 41 66.5) (end 35.5 66.5) (width 1) (layer B.Cu) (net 1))
 (segment (start 33.38 64.38) (end 33.38 60.62) (width 1) (layer B.Cu) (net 1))
 (segment (start 35.5 66.5) (end 33.38 64.38) (width 1) (layer B.Cu) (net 1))
 (segment (start 35.5 66.5) (end 32.5 66.5) (width 1) (layer B.Cu) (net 1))
 (segment (start 30.84 64.84) (end 30.84 60.62) (width 1) (layer B.Cu) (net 1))
 (segment (start 32.5 66.5) (end 30.84 64.84) (width 1) (layer B.Cu) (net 1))
 (segment (start 144.5 46) (end 147 46) (width 1) (layer F.Cu) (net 1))
 (segment (start 147 47.5) (end 150 50.5) (width 1) (layer F.Cu) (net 1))
 (segment (start 147 46) (end 147 47.5) (width 1) (layer F.Cu) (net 1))
 (segment (start 88 105.5) (end 88 101.5) (width 1) (layer B.Cu) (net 1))
 (segment (start 85 108.5) (end 88 105.5) (width 1) (layer B.Cu) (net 1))
 (segment (start 54 108.5) (end 85 108.5) (width 1) (layer B.Cu) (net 1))
 (segment (start 53 107.5) (end 54 108.5) (width 1) (layer B.Cu) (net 1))
 (segment (start 53 105.5) (end 53 107.5) (width 1) (layer B.Cu) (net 1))
 (segment (start 41 66.5) (end 41 106.5) (width 1) (layer B.Cu) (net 1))
 (segment (start 32.5 66.5) (end 29 66.5) (width 1) (layer B.Cu) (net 1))
 (segment (start 23.22 60.62) (end 23.22 62.72) (width 1) (layer B.Cu) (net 1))
 (segment (start 27 66.5) (end 29 66.5) (width 1) (layer B.Cu) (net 1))
 (segment (start 23.22 62.72) (end 27 66.5) (width 1) (layer B.Cu) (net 1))
 (segment (start 140.949999 81.989999) (end 140.949999 81.050001) (width 1) (layer B.Cu) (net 1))
 (segment (start 140.949999 81.050001) (end 142.5 79.5) (width 1) (layer B.Cu) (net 1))
 (segment (start 142.5 79.5) (end 142.5 73) (width 1) (layer B.Cu) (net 1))
 (segment (start 38.5 86.5) (end 47.56 86.5) (width 1) (layer F.Cu) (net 10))
 (segment (start 23.22 101.78) (end 38.5 86.5) (width 1) (layer F.Cu) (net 10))
 (segment (start 23.22 106.5) (end 23.22 101.78) (width 1) (layer F.Cu) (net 10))
 (segment (start 112.479114 67.991773) (end 112.479114 75.520886) (width 1) (layer F.Cu) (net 10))
 (segment (start 112.479114 75.520886) (end 106 82) (width 1) (layer F.Cu) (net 10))
 (segment (start 106 82) (end 101 82) (width 1) (layer F.Cu) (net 10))
 (segment (start 49.5 86.5) (end 47.56 86.5) (width 1) (layer F.Cu) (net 10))
 (segment (start 54 82) (end 49.5 86.5) (width 1) (layer F.Cu) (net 10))
 (segment (start 101 82) (end 54 82) (width 1) (layer F.Cu) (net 10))
 (via (at 101 82) (size 2) (drill 1) (layers F.Cu B.Cu) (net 10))
 (segment (start 143.3 99.2) (end 148 99.2) (width 1) (layer B.Cu) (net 10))
 (segment (start 137 105.5) (end 143.3 99.2) (width 1) (layer B.Cu) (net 10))
 (segment (start 122.5 105.5) (end 137 105.5) (width 1) (layer B.Cu) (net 10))
 (segment (start 101 84) (end 122.5 105.5) (width 1) (layer B.Cu) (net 10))
 (segment (start 101 82) (end 101 84) (width 1) (layer B.Cu) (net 10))
 (segment (start 41 60.62) (end 41 62) (width 1) (layer F.Cu) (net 10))
 (segment (start 38.5 64.5) (end 38.5 86.5) (width 1) (layer F.Cu) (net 10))
 (segment (start 41 62) (end 38.5 64.5) (width 1) (layer F.Cu) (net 10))
 (segment (start 41 53) (end 41 60.5) (width 1) (layer F.Cu) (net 10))
 (segment (start 28.3 53) (end 28.3 51.8) (width 1) (layer B.Cu) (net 40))
 (segment (start 25.5 49) (end 25.5 46) (width 1) (layer B.Cu) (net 40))
 (segment (start 28.3 51.8) (end 25.5 49) (width 1) (layer B.Cu) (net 40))
 (segment (start 35.92 53) (end 35.92 51.42) (width 1) (layer B.Cu) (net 41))
 (segment (start 35.92 51.42) (end 34.5 50) (width 1) (layer B.Cu) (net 41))
 (segment (start 32 50) (end 28 46) (width 1) (layer B.Cu) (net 41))
 (segment (start 34.5 50) (end 32 50) (width 1) (layer B.Cu) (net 41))
 (segment (start 55.5 101.42) (end 70.42 86.5) (width 1) (layer B.Cu) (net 33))
 (segment (start 55.5 105.5) (end 55.5 101.42) (width 1) (layer B.Cu) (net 33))
 (segment (start 47.56 83.5) (end 43.5 79.44) (width 1) (layer F.Cu) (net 32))
 (segment (start 43.5 50.5) (end 39 46) (width 1) (layer F.Cu) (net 32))
 (segment (start 43.5 79.44) (end 43.5 50.5) (width 1) (layer F.Cu) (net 32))
 (segment (start 47.56 75.5) (end 46 75.5) (width 1) (layer F.Cu) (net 31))
 (segment (start 46 75.5) (end 45.5 75) (width 1) (layer F.Cu) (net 31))
 (segment (start 45.5 75) (end 45.5 46.5) (width 1) (layer F.Cu) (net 31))
 (segment (start 45.5 46.5) (end 42.5 43.5) (width 1) (layer F.Cu) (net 31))
 (segment (start 42.5 43.5) (end 38 43.5) (width 1) (layer F.Cu) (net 31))
 (segment (start 36.5 45) (end 38 43.5) (width 1) (layer F.Cu) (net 31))
 (segment (start 36.5 46) (end 36.5 45) (width 1) (layer F.Cu) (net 31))
 (segment (start 148 96.66) (end 150 94.66) (width 1) (layer B.Cu) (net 2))
 (segment (start 150 94.66) (end 150 82.5) (width 1) (layer B.Cu) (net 2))
 (segment (start 150 82.5) (end 147 79.5) (width 1) (layer B.Cu) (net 2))
 (segment (start 147 79.5) (end 147 73) (width 1) (layer B.Cu) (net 2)))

